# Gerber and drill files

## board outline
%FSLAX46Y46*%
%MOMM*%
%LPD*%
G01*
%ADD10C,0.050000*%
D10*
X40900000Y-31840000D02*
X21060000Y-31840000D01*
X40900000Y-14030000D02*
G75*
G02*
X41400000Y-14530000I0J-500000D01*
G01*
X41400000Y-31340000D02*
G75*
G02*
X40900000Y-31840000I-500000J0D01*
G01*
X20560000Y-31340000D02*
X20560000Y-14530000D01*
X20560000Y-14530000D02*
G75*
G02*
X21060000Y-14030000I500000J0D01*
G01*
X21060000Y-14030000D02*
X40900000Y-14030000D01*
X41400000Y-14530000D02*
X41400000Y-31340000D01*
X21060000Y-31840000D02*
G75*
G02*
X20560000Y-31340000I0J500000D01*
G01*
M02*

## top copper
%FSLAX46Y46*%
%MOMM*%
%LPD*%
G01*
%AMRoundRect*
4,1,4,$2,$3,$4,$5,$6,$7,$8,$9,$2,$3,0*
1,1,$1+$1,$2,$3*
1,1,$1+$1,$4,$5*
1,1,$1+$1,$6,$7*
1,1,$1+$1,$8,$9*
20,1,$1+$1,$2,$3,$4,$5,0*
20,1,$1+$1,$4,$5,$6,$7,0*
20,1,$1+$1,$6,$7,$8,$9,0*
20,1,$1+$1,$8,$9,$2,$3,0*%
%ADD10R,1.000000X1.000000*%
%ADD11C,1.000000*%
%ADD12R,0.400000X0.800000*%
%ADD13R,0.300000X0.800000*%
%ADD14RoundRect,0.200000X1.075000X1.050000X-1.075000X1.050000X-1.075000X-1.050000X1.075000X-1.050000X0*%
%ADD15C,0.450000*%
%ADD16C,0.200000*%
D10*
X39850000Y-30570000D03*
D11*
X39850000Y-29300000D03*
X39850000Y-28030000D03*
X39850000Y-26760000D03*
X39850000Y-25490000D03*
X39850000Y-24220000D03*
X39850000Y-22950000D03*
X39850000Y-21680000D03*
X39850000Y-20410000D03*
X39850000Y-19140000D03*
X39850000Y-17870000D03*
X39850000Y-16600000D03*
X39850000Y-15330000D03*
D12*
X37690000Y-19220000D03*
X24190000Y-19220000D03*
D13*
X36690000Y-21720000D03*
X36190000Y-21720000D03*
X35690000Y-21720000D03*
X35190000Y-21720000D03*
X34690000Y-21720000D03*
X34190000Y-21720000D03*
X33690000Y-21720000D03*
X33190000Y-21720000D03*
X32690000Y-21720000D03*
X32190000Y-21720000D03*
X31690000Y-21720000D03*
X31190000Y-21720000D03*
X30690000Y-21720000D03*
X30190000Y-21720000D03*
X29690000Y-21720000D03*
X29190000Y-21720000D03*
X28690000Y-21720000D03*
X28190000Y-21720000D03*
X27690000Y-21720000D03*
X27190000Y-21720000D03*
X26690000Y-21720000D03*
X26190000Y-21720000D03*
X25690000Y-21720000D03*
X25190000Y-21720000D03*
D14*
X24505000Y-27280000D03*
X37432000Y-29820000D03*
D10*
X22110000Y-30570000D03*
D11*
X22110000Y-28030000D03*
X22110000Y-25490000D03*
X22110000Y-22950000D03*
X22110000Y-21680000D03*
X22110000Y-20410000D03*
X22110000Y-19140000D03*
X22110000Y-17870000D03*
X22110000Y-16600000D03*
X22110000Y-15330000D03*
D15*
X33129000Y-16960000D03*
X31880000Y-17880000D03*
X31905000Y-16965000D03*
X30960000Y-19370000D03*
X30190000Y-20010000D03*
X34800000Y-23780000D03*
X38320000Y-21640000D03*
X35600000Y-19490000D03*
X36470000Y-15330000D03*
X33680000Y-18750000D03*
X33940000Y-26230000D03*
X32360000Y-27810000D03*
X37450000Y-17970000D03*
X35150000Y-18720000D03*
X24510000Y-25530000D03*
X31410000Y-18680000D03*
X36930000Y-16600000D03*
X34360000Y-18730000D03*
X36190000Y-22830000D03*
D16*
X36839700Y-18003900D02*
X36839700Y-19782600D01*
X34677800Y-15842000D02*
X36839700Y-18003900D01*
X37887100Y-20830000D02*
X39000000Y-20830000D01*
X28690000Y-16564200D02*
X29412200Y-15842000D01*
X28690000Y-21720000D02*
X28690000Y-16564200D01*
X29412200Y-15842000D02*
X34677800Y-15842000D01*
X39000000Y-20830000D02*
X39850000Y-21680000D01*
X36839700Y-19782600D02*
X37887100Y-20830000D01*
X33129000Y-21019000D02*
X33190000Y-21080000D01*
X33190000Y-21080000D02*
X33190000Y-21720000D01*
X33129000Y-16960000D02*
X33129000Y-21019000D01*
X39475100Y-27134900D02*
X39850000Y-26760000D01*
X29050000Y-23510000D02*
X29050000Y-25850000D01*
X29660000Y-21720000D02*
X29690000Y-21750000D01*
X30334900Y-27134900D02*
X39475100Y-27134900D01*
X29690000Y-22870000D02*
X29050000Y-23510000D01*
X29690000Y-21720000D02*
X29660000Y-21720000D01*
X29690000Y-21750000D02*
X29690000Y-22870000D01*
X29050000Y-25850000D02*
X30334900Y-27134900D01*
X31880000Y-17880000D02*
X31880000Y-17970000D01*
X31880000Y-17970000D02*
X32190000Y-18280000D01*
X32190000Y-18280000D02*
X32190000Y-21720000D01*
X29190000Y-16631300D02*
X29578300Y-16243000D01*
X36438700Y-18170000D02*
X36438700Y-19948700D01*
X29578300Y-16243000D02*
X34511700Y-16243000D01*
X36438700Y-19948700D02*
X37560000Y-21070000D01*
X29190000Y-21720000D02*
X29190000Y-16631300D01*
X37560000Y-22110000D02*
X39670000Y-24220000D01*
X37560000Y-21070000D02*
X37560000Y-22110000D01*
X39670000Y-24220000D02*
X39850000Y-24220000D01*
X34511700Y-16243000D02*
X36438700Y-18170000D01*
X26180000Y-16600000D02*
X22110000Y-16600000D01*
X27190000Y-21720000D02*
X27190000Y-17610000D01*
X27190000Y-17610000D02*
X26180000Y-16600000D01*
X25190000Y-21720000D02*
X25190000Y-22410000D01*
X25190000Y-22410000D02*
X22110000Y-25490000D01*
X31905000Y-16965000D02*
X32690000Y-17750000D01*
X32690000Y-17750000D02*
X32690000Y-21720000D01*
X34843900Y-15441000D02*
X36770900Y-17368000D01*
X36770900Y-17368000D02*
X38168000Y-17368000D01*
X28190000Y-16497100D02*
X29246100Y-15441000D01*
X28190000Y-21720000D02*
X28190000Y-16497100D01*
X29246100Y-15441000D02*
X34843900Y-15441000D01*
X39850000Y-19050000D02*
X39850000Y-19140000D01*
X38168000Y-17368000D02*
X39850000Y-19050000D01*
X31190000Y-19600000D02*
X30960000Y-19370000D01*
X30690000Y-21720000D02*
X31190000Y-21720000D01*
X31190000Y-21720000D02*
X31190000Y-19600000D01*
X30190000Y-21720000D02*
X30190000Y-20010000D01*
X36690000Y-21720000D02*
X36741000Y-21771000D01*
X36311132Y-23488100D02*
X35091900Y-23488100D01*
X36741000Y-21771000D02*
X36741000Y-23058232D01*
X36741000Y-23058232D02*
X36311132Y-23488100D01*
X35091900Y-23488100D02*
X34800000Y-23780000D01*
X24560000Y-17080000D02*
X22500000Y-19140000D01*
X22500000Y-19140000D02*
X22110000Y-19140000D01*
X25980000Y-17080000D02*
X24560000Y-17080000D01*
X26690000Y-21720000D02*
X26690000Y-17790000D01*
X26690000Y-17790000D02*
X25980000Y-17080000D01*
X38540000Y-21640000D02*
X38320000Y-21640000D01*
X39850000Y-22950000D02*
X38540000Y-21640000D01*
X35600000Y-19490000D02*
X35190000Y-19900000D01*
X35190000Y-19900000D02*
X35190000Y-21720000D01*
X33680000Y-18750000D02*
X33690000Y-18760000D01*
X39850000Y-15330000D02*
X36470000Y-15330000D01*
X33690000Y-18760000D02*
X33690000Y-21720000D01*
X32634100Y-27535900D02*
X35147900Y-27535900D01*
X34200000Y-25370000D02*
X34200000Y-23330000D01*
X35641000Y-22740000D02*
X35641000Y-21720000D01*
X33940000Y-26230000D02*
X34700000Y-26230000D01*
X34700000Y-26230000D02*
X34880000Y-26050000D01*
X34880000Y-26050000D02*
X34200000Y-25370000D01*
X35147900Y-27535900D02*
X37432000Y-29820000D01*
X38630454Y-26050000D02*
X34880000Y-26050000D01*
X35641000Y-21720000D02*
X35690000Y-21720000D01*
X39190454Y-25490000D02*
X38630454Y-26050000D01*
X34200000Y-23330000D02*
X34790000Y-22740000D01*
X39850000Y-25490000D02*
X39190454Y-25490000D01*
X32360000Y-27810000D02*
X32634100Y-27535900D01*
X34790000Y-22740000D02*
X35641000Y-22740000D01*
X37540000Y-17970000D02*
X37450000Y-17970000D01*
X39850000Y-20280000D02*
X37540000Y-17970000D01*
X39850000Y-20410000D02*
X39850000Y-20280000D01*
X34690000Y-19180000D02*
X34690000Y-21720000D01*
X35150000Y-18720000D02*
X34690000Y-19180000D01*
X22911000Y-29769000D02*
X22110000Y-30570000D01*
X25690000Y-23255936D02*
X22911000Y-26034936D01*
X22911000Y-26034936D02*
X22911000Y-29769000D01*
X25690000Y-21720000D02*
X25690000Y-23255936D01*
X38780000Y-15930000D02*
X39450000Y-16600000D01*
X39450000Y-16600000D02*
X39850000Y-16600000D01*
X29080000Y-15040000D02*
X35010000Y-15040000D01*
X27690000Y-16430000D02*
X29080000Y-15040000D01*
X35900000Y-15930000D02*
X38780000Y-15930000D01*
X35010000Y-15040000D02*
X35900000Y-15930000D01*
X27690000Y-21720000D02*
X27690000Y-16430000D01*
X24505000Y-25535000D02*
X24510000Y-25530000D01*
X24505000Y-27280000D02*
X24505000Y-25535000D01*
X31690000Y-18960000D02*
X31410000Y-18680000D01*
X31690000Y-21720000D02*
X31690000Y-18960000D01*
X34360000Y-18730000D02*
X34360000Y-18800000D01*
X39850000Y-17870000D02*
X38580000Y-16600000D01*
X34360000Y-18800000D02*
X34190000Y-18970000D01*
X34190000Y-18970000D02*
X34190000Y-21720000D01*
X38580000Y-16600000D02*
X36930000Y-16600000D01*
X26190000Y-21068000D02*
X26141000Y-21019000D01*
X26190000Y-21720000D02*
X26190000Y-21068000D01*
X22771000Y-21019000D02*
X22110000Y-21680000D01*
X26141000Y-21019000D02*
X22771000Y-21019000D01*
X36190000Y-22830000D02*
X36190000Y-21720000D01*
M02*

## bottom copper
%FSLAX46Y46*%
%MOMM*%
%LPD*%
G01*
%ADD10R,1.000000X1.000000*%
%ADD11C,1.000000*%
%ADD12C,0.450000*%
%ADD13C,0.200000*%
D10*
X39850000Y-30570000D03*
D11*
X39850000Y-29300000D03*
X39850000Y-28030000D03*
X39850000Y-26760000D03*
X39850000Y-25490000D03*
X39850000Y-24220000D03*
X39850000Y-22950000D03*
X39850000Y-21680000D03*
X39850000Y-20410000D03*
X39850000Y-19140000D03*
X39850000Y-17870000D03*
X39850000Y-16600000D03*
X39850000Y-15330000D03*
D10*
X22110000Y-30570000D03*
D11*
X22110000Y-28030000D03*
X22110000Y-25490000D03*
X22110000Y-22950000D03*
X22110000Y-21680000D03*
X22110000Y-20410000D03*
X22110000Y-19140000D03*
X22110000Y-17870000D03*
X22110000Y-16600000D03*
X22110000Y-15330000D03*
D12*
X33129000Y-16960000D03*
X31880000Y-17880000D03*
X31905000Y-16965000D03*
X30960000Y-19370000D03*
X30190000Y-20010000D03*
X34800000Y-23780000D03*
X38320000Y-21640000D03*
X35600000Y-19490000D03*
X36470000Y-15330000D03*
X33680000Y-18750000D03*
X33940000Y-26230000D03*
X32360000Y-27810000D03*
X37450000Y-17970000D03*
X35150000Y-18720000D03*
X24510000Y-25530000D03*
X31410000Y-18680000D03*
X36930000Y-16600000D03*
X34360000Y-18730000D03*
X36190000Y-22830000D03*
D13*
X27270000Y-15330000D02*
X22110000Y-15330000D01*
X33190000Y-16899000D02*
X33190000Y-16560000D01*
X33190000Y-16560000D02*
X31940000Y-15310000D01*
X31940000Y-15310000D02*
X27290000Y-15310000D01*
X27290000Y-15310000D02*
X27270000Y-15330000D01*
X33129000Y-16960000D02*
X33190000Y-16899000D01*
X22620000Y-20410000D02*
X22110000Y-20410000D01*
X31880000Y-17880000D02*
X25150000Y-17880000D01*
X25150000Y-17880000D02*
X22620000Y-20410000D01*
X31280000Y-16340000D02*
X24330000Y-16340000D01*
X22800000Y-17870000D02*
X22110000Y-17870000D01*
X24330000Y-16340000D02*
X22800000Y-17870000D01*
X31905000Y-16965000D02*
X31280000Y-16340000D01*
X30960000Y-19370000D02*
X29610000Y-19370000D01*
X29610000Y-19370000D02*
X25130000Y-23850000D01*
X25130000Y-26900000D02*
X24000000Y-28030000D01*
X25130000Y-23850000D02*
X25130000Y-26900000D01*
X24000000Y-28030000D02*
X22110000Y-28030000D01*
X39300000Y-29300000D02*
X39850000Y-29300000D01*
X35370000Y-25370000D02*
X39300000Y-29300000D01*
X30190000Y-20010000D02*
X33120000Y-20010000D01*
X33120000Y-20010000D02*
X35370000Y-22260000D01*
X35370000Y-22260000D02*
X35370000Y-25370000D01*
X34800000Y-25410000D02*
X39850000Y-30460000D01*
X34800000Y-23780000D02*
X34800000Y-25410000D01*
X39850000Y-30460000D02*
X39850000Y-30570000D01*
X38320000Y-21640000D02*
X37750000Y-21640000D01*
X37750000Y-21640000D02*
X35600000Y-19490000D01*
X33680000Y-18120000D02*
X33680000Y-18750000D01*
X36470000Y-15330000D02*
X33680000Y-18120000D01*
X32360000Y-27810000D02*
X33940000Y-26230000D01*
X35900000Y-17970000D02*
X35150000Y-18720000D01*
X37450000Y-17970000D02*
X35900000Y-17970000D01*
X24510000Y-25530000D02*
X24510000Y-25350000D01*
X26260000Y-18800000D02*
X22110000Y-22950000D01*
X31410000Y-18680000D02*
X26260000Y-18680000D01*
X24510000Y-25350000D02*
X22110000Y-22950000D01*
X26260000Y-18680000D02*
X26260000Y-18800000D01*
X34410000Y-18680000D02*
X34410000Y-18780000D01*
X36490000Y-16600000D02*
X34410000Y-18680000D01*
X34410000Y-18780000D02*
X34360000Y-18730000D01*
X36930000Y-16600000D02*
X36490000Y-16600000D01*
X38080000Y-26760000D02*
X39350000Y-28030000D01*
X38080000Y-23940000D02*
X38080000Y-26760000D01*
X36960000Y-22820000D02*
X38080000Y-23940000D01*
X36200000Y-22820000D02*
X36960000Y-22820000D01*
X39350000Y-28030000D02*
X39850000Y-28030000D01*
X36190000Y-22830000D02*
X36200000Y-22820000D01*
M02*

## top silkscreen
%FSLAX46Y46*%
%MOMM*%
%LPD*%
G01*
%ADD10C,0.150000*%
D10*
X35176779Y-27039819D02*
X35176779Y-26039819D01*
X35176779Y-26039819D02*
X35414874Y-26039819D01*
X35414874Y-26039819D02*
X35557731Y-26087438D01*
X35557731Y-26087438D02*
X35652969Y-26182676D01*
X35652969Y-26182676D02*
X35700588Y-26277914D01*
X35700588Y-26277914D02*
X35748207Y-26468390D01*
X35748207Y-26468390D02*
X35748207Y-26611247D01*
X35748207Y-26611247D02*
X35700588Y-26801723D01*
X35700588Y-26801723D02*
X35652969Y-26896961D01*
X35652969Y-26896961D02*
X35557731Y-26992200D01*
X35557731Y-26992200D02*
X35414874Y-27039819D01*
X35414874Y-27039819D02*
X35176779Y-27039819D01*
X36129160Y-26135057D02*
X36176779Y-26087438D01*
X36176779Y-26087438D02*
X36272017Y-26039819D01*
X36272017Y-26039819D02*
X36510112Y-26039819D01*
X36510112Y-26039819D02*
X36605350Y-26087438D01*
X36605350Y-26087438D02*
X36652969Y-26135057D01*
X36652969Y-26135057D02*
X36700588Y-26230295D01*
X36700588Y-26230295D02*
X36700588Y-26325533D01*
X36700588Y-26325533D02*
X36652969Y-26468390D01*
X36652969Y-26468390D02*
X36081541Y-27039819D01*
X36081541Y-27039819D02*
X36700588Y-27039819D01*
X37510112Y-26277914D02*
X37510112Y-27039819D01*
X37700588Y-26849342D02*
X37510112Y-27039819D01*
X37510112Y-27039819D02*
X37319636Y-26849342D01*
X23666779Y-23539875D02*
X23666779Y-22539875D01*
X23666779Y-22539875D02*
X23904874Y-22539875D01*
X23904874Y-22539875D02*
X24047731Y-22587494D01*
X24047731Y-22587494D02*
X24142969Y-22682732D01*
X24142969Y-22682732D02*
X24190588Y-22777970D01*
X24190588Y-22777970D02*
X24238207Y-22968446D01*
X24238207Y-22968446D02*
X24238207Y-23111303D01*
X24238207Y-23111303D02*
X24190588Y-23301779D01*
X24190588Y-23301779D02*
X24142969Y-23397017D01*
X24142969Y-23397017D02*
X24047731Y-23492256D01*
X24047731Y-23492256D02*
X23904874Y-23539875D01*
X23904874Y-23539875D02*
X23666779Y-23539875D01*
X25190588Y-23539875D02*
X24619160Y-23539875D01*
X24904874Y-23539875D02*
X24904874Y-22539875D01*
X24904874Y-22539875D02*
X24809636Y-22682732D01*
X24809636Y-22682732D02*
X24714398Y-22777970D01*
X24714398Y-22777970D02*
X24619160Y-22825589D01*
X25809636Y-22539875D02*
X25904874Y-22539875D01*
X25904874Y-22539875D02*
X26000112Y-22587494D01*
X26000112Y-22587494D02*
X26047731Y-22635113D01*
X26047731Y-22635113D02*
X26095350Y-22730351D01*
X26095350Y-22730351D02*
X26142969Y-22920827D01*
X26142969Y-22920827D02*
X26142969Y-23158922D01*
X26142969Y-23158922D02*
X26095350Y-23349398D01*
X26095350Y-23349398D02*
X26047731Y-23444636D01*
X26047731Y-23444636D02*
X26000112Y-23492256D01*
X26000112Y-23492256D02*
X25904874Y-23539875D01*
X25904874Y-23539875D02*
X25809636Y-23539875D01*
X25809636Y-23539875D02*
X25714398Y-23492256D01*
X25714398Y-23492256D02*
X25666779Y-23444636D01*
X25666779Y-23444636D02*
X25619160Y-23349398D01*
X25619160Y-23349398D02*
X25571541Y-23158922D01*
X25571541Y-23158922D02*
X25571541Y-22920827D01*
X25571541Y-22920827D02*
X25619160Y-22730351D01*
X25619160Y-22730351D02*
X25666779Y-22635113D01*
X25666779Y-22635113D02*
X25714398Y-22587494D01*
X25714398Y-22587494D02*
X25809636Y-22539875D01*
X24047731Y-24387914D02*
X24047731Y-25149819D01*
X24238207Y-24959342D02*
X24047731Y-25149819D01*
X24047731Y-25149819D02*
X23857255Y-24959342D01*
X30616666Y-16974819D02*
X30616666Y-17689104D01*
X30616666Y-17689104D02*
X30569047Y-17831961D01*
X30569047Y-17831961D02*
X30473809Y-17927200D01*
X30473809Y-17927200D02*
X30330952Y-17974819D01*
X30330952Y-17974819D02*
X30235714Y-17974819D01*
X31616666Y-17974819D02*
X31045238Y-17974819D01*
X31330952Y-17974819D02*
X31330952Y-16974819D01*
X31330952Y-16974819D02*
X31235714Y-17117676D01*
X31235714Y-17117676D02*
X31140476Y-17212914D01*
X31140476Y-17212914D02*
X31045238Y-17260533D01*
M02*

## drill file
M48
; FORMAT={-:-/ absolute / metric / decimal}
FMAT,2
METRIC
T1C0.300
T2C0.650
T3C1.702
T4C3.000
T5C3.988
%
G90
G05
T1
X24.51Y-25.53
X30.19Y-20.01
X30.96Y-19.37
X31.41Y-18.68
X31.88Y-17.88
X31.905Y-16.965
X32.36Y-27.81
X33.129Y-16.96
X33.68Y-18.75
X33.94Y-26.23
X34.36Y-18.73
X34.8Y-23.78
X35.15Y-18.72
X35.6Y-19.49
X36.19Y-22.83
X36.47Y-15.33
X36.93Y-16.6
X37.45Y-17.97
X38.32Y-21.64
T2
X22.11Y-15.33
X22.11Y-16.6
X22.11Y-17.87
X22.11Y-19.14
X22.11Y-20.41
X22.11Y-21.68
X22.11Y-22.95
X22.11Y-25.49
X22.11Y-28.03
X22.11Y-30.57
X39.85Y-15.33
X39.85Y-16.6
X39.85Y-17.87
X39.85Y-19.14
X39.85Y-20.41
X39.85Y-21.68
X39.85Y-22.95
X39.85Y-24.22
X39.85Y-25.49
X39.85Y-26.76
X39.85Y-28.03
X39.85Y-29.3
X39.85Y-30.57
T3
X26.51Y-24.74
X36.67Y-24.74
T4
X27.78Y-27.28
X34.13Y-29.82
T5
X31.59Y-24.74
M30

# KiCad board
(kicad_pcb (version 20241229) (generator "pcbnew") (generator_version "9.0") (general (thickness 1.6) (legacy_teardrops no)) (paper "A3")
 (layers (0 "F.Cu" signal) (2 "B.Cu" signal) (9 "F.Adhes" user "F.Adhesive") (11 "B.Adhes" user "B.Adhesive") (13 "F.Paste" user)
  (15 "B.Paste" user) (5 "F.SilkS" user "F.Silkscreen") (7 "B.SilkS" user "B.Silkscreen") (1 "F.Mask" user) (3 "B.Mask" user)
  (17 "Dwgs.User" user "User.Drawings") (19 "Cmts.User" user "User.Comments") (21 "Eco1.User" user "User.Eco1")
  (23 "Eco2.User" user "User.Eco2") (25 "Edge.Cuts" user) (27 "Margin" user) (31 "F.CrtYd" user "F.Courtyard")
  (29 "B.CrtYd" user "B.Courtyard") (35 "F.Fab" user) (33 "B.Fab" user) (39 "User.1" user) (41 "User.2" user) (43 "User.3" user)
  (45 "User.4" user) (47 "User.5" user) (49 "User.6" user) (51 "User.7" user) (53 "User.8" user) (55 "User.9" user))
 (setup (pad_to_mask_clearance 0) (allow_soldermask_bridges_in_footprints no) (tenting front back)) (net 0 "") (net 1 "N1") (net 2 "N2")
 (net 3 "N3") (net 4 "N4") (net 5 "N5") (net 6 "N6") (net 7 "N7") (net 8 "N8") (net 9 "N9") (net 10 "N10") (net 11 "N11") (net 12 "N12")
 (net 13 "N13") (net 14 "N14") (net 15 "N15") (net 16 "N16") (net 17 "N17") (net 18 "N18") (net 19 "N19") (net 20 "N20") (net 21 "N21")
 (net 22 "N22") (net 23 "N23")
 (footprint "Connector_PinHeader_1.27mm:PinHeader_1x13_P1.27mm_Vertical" (layer "F.Cu") (at 39.85 30.57 180)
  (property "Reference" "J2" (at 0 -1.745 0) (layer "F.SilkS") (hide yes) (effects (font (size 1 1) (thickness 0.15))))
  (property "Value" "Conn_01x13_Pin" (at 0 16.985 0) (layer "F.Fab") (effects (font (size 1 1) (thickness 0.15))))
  (pad "1" thru_hole rect (at 0 0 180) (size 1 1) (drill 0.65) (layers "*.Cu" "*.Mask") (remove_unused_layers no) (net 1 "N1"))
  (pad "2" thru_hole circle (at 0 1.27 180) (size 1 1) (drill 0.65) (layers "*.Cu" "*.Mask") (remove_unused_layers no) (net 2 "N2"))
  (pad "3" thru_hole circle (at 0 2.54 180) (size 1 1) (drill 0.65) (layers "*.Cu" "*.Mask") (remove_unused_layers no) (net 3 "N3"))
  (pad "4" thru_hole circle (at 0 3.81 180) (size 1 1) (drill 0.65) (layers "*.Cu" "*.Mask") (remove_unused_layers no) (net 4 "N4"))
  (pad "5" thru_hole circle (at 0 5.08 180) (size 1 1) (drill 0.65) (layers "*.Cu" "*.Mask") (remove_unused_layers no) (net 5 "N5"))
  (pad "6" thru_hole circle (at 0 6.35 180) (size 1 1) (drill 0.65) (layers "*.Cu" "*.Mask") (remove_unused_layers no) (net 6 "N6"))
  (pad "7" thru_hole circle (at 0 7.62 180) (size 1 1) (drill 0.65) (layers "*.Cu" "*.Mask") (remove_unused_layers no) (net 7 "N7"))
  (pad "8" thru_hole circle (at 0 8.89 180) (size 1 1) (drill 0.65) (layers "*.Cu" "*.Mask") (remove_unused_layers no) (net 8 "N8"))
  (pad "9" thru_hole circle (at 0 10.16 180) (size 1 1) (drill 0.65) (layers "*.Cu" "*.Mask") (remove_unused_layers no) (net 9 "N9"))
  (pad "10" thru_hole circle (at 0 11.43 180) (size 1 1) (drill 0.65) (layers "*.Cu" "*.Mask") (remove_unused_layers no) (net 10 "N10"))
  (pad "11" thru_hole circle (at 0 12.7 180) (size 1 1) (drill 0.65) (layers "*.Cu" "*.Mask") (remove_unused_layers no) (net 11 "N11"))
  (pad "12" thru_hole circle (at 0 13.97 180) (size 1 1) (drill 0.65) (layers "*.Cu" "*.Mask") (remove_unused_layers no) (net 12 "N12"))
  (pad "13" thru_hole circle (at 0 15.24 180) (size 1 1) (drill 0.65) (layers "*.Cu" "*.Mask") (remove_unused_layers no) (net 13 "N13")))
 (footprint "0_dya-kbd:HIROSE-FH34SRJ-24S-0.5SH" (layer "F.Cu") (at 30.94 21.72 180)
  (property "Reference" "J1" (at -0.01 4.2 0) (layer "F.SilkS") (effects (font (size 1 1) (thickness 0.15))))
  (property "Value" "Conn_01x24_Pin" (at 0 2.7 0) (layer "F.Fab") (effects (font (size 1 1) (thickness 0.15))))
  (pad "0" smd rect (at -6.75 2.5 180) (size 0.4 0.8) (layers "F.Cu" "F.Mask" "F.Paste") (thermal_bridge_angle 45))
  (pad "0" smd rect (at 6.75 2.5 180) (size 0.4 0.8) (layers "F.Cu" "F.Mask" "F.Paste") (thermal_bridge_angle 45))
  (pad "1" smd rect (at -5.75 0 180) (size 0.3 0.8) (layers "F.Cu" "F.Mask" "F.Paste") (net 1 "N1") (thermal_bridge_angle 45))
  (pad "2" smd rect (at -5.25 0 180) (size 0.3 0.8) (layers "F.Cu" "F.Mask" "F.Paste") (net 3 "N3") (thermal_bridge_angle 45))
  (pad "3" smd rect (at -4.75 0 180) (size 0.3 0.8) (layers "F.Cu" "F.Mask" "F.Paste") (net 5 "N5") (thermal_bridge_angle 45))
  (pad "4" smd rect (at -4.25 0 180) (size 0.3 0.8) (layers "F.Cu" "F.Mask" "F.Paste") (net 7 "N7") (thermal_bridge_angle 45))
  (pad "5" smd rect (at -3.75 0 180) (size 0.3 0.8) (layers "F.Cu" "F.Mask" "F.Paste") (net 9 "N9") (thermal_bridge_angle 45))
  (pad "6" smd rect (at -3.25 0 180) (size 0.3 0.8) (layers "F.Cu" "F.Mask" "F.Paste") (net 11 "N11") (thermal_bridge_angle 45))
  (pad "7" smd rect (at -2.75 0 180) (size 0.3 0.8) (layers "F.Cu" "F.Mask" "F.Paste") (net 13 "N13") (thermal_bridge_angle 45))
  (pad "8" smd rect (at -2.25 0 180) (size 0.3 0.8) (layers "F.Cu" "F.Mask" "F.Paste") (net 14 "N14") (thermal_bridge_angle 45))
  (pad "9" smd rect (at -1.75 0 180) (size 0.3 0.8) (layers "F.Cu" "F.Mask" "F.Paste") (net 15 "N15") (thermal_bridge_angle 45))
  (pad "10" smd rect (at -1.25 0 180) (size 0.3 0.8) (layers "F.Cu" "F.Mask" "F.Paste") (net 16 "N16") (thermal_bridge_angle 45))
  (pad "11" smd rect (at -0.75 0 180) (size 0.3 0.8) (layers "F.Cu" "F.Mask" "F.Paste") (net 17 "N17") (thermal_bridge_angle 45))
  (pad "12" smd rect (at -0.25 0 180) (size 0.3 0.8) (layers "F.Cu" "F.Mask" "F.Paste") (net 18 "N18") (thermal_bridge_angle 45))
  (pad "13" smd rect (at 0.25 0 180) (size 0.3 0.8) (layers "F.Cu" "F.Mask" "F.Paste") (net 18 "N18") (thermal_bridge_angle 45))
  (pad "14" smd rect (at 0.75 0 180) (size 0.3 0.8) (layers "F.Cu" "F.Mask" "F.Paste") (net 2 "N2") (thermal_bridge_angle 45))
  (pad "15" smd rect (at 1.25 0 180) (size 0.3 0.8) (layers "F.Cu" "F.Mask" "F.Paste") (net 4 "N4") (thermal_bridge_angle 45))
  (pad "16" smd rect (at 1.75 0 180) (size 0.3 0.8) (layers "F.Cu" "F.Mask" "F.Paste") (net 6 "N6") (thermal_bridge_angle 45))
  (pad "17" smd rect (at 2.25 0 180) (size 0.3 0.8) (layers "F.Cu" "F.Mask" "F.Paste") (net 8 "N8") (thermal_bridge_angle 45))
  (pad "18" smd rect (at 2.75 0 180) (size 0.3 0.8) (layers "F.Cu" "F.Mask" "F.Paste") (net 10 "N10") (thermal_bridge_angle 45))
  (pad "19" smd rect (at 3.25 0 180) (size 0.3 0.8) (layers "F.Cu" "F.Mask" "F.Paste") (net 12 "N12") (thermal_bridge_angle 45))
  (pad "20" smd rect (at 3.75 0 180) (size 0.3 0.8) (layers "F.Cu" "F.Mask" "F.Paste") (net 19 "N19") (thermal_bridge_angle 45))
  (pad "21" smd rect (at 4.25 0 180) (size 0.3 0.8) (layers "F.Cu" "F.Mask" "F.Paste") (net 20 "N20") (thermal_bridge_angle 45))
  (pad "22" smd rect (at 4.75 0 180) (size 0.3 0.8) (layers "F.Cu" "F.Mask" "F.Paste") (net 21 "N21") (thermal_bridge_angle 45))
  (pad "23" smd rect (at 5.25 0 180) (size 0.3 0.8) (layers "F.Cu" "F.Mask" "F.Paste") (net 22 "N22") (thermal_bridge_angle 45))
  (pad "24" smd rect (at 5.75 0 180) (size 0.3 0.8) (layers "F.Cu" "F.Mask" "F.Paste") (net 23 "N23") (thermal_bridge_angle 45)))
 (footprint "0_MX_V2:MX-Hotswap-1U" (layer "F.Cu") (at 31.59 24.74 180)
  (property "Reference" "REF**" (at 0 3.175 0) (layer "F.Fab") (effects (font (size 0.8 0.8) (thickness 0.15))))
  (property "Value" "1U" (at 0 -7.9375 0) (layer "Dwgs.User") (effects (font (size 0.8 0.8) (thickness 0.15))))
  (pad "" np_thru_hole circle (at -5.08 0 131.901) (size 1.7018 1.7018) (drill 1.7018) (layers "*.Cu" "*.Mask"))
  (pad "" np_thru_hole circle (at -2.54 -5.08 180) (size 3 3) (drill 3) (layers "*.Cu" "*.Mask"))
  (pad "" np_thru_hole circle (at 0 0 180) (size 3.9878 3.9878) (drill 3.9878) (layers "*.Cu" "*.Mask"))
  (pad "" np_thru_hole circle (at 3.81 -2.54 180) (size 3 3) (drill 3) (layers "*.Cu" "*.Mask"))
  (pad "" np_thru_hole circle (at 5.08 0 131.901) (size 1.7018 1.7018) (drill 1.7018) (layers "*.Cu" "*.Mask"))
  (pad "1" smd roundrect (at 7.085 -2.54 180) (size 2.55 2.5) (layers "F.Cu" "F.Mask" "F.Paste") (roundrect_rratio 0.08) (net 17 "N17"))
  (pad "2" smd roundrect (at -5.842 -5.08 180) (size 2.55 2.5) (layers "F.Cu" "F.Mask" "F.Paste") (roundrect_rratio 0.08) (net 5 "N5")))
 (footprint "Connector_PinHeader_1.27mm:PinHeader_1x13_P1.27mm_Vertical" (layer "F.Cu") (at 22.11 30.57 180)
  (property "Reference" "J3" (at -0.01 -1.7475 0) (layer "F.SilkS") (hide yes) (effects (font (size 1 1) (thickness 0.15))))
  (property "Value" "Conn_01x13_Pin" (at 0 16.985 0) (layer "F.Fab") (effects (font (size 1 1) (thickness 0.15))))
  (pad "1" thru_hole rect (at 0 0 180) (size 1 1) (drill 0.65) (layers "*.Cu" "*.Mask") (remove_unused_layers no) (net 22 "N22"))
  (pad "3" thru_hole circle (at 0 2.54 180) (size 1 1) (drill 0.65) (layers "*.Cu" "*.Mask") (remove_unused_layers no) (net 18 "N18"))
  (pad "5" thru_hole circle (at 0 5.08 180) (size 1 1) (drill 0.65) (layers "*.Cu" "*.Mask") (remove_unused_layers no) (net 23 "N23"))
  (pad "7" thru_hole circle (at 0 7.62 180) (size 1 1) (drill 0.65) (layers "*.Cu" "*.Mask") (remove_unused_layers no) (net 17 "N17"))
  (pad "8" thru_hole circle (at 0 8.89 180) (size 1 1) (drill 0.65) (layers "*.Cu" "*.Mask") (remove_unused_layers no) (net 21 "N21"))
  (pad "9" thru_hole circle (at 0 10.16 180) (size 1 1) (drill 0.65) (layers "*.Cu" "*.Mask") (remove_unused_layers no) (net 16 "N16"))
  (pad "10" thru_hole circle (at 0 11.43 180) (size 1 1) (drill 0.65) (layers "*.Cu" "*.Mask") (remove_unused_layers no) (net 20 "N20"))
  (pad "11" thru_hole circle (at 0 12.7 180) (size 1 1) (drill 0.65) (layers "*.Cu" "*.Mask") (remove_unused_layers no) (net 15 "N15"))
  (pad "12" thru_hole circle (at 0 13.97 180) (size 1 1) (drill 0.65) (layers "*.Cu" "*.Mask") (remove_unused_layers no) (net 19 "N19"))
  (pad "13" thru_hole circle (at 0 15.24 180) (size 1 1) (drill 0.65) (layers "*.Cu" "*.Mask") (remove_unused_layers no) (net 14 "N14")))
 (gr_line (start 40.9 31.84) (end 21.06 31.84) (stroke (width 0.05) (type default)) (layer "Edge.Cuts"))
 (gr_arc (start 40.9 14.03) (mid 41.253553 14.176447) (end 41.4 14.53) (stroke (width 0.05) (type default)) (layer "Edge.Cuts"))
 (gr_arc (start 41.4 31.34) (mid 41.253553 31.693553) (end 40.9 31.84) (stroke (width 0.05) (type default)) (layer "Edge.Cuts"))
 (gr_line (start 20.56 31.34) (end 20.56 14.53) (stroke (width 0.05) (type default)) (layer "Edge.Cuts"))
 (gr_arc (start 20.56 14.53) (mid 20.706447 14.176447) (end 21.06 14.03) (stroke (width 0.05) (type default)) (layer "Edge.Cuts"))
 (gr_line (start 21.06 14.03) (end 40.9 14.03) (stroke (width 0.05) (type default)) (layer "Edge.Cuts"))
 (gr_line (start 41.4 14.53) (end 41.4 31.34) (stroke (width 0.05) (type default)) (layer "Edge.Cuts"))
 (gr_arc (start 21.06 31.84) (mid 20.706447 31.693553) (end 20.56 31.34) (stroke (width 0.05) (type default)) (layer "Edge.Cuts"))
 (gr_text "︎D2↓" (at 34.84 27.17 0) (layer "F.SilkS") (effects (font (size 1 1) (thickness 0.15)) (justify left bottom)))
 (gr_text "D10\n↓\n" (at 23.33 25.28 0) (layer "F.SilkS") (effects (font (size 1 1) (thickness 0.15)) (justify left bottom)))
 (segment (start 36.8397 18.0039) (end 36.8397 19.7826) (width 0.2) (layer "F.Cu") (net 8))
 (segment (start 34.6778 15.842) (end 36.8397 18.0039) (width 0.2) (layer "F.Cu") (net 8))
 (segment (start 37.8871 20.83) (end 39 20.83) (width 0.2) (layer "F.Cu") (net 8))
 (segment (start 28.69 16.5642) (end 29.4122 15.842) (width 0.2) (layer "F.Cu") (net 8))
 (segment (start 28.69 21.72) (end 28.69 16.5642) (width 0.2) (layer "F.Cu") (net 8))
 (segment (start 29.4122 15.842) (end 34.6778 15.842) (width 0.2) (layer "F.Cu") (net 8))
 (segment (start 39 20.83) (end 39.85 21.68) (width 0.2) (layer "F.Cu") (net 8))
 (segment (start 36.8397 19.7826) (end 37.8871 20.83) (width 0.2) (layer "F.Cu") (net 8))
 (segment (start 33.129 21.019) (end 33.19 21.08) (width 0.2) (layer "F.Cu") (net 14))
 (segment (start 33.19 21.08) (end 33.19 21.72) (width 0.2) (layer "F.Cu") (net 14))
 (segment (start 33.129 16.96) (end 33.129 21.019) (width 0.2) (layer "F.Cu") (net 14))
 (via (at 33.129 16.96) (size 0.45) (drill 0.3) (layers "F.Cu" "B.Cu") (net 14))
 (segment (start 27.27 15.33) (end 22.11 15.33) (width 0.2) (layer "B.Cu") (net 14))
 (segment (start 33.19 16.899) (end 33.19 16.56) (width 0.2) (layer "B.Cu") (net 14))
 (segment (start 33.19 16.56) (end 31.94 15.31) (width 0.2) (layer "B.Cu") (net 14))
 (segment (start 31.94 15.31) (end 27.29 15.31) (width 0.2) (layer "B.Cu") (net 14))
 (segment (start 27.29 15.31) (end 27.27 15.33) (width 0.2) (layer "B.Cu") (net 14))
 (segment (start 33.129 16.96) (end 33.19 16.899) (width 0.2) (layer "B.Cu") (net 14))
 (segment (start 39.4751 27.1349) (end 39.85 26.76) (width 0.2) (layer "F.Cu") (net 4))
 (segment (start 29.05 23.51) (end 29.05 25.85) (width 0.2) (layer "F.Cu") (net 4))
 (segment (start 29.66 21.72) (end 29.69 21.75) (width 0.2) (layer "F.Cu") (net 4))
 (segment (start 30.3349 27.1349) (end 39.4751 27.1349) (width 0.2) (layer "F.Cu") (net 4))
 (segment (start 29.69 22.87) (end 29.05 23.51) (width 0.2) (layer "F.Cu") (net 4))
 (segment (start 29.69 21.72) (end 29.66 21.72) (width 0.2) (layer "F.Cu") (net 4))
 (segment (start 29.69 21.75) (end 29.69 22.87) (width 0.2) (layer "F.Cu") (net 4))
 (segment (start 29.05 25.85) (end 30.3349 27.1349) (width 0.2) (layer "F.Cu") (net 4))
 (segment (start 31.88 17.88) (end 31.88 17.97) (width 0.2) (layer "F.Cu") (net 16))
 (segment (start 31.88 17.97) (end 32.19 18.28) (width 0.2) (layer "F.Cu") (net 16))
 (segment (start 32.19 18.28) (end 32.19 21.72) (width 0.2) (layer "F.Cu") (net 16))
 (via (at 31.88 17.88) (size 0.45) (drill 0.3) (layers "F.Cu" "B.Cu") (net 16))
 (segment (start 22.62 20.41) (end 22.11 20.41) (width 0.2) (layer "B.Cu") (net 16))
 (segment (start 31.88 17.88) (end 25.15 17.88) (width 0.2) (layer "B.Cu") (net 16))
 (segment (start 25.15 17.88) (end 22.62 20.41) (width 0.2) (layer "B.Cu") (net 16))
 (segment (start 29.19 16.6313) (end 29.5783 16.243) (width 0.2) (layer "F.Cu") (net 6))
 (segment (start 36.4387 18.17) (end 36.4387 19.9487) (width 0.2) (layer "F.Cu") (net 6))
 (segment (start 29.5783 16.243) (end 34.5117 16.243) (width 0.2) (layer "F.Cu") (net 6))
 (segment (start 36.4387 19.9487) (end 37.56 21.07) (width 0.2) (layer "F.Cu") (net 6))
 (segment (start 29.19 21.72) (end 29.19 16.6313) (width 0.2) (layer "F.Cu") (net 6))
 (segment (start 37.56 22.11) (end 39.67 24.22) (width 0.2) (layer "F.Cu") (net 6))
 (segment (start 37.56 21.07) (end 37.56 22.11) (width 0.2) (layer "F.Cu") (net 6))
 (segment (start 39.67 24.22) (end 39.85 24.22) (width 0.2) (layer "F.Cu") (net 6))
 (segment (start 34.5117 16.243) (end 36.4387 18.17) (width 0.2) (layer "F.Cu") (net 6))
 (segment (start 26.18 16.6) (end 22.11 16.6) (width 0.2) (layer "F.Cu") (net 19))
 (segment (start 27.19 21.72) (end 27.19 17.61) (width 0.2) (layer "F.Cu") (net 19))
 (segment (start 27.19 17.61) (end 26.18 16.6) (width 0.2) (layer "F.Cu") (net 19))
 (segment (start 25.19 21.72) (end 25.19 22.41) (width 0.2) (layer "F.Cu") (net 23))
 (segment (start 25.19 22.41) (end 22.11 25.49) (width 0.2) (layer "F.Cu") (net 23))
 (segment (start 31.905 16.965) (end 32.69 17.75) (width 0.2) (layer "F.Cu") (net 15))
 (segment (start 32.69 17.75) (end 32.69 21.72) (width 0.2) (layer "F.Cu") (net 15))
 (via (at 31.905 16.965) (size 0.45) (drill 0.3) (layers "F.Cu" "B.Cu") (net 15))
 (segment (start 31.28 16.34) (end 24.33 16.34) (width 0.2) (layer "B.Cu") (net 15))
 (segment (start 22.8 17.87) (end 22.11 17.87) (width 0.2) (layer "B.Cu") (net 15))
 (segment (start 24.33 16.34) (end 22.8 17.87) (width 0.2) (layer "B.Cu") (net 15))
 (segment (start 31.905 16.965) (end 31.28 16.34) (width 0.2) (layer "B.Cu") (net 15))
 (segment (start 34.8439 15.441) (end 36.7709 17.368) (width 0.2) (layer "F.Cu") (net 10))
 (segment (start 36.7709 17.368) (end 38.168 17.368) (width 0.2) (layer "F.Cu") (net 10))
 (segment (start 28.19 16.4971) (end 29.2461 15.441) (width 0.2) (layer "F.Cu") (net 10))
 (segment (start 28.19 21.72) (end 28.19 16.4971) (width 0.2) (layer "F.Cu") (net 10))
 (segment (start 29.2461 15.441) (end 34.8439 15.441) (width 0.2) (layer "F.Cu") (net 10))
 (segment (start 39.85 19.05) (end 39.85 19.14) (width 0.2) (layer "F.Cu") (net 10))
 (segment (start 38.168 17.368) (end 39.85 19.05) (width 0.2) (layer "F.Cu") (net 10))
 (segment (start 31.19 19.6) (end 30.96 19.37) (width 0.2) (layer "F.Cu") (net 18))
 (segment (start 30.69 21.72) (end 31.19 21.72) (width 0.2) (layer "F.Cu") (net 18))
 (segment (start 31.19 21.72) (end 31.19 19.6) (width 0.2) (layer "F.Cu") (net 18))
 (via (at 30.96 19.37) (size 0.45) (drill 0.3) (layers "F.Cu" "B.Cu") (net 18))
 (segment (start 30.96 19.37) (end 29.61 19.37) (width 0.2) (layer "B.Cu") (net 18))
 (segment (start 29.61 19.37) (end 25.13 23.85) (width 0.2) (layer "B.Cu") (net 18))
 (segment (start 25.13 26.9) (end 24 28.03) (width 0.2) (layer "B.Cu") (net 18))
 (segment (start 25.13 23.85) (end 25.13 26.9) (width 0.2) (layer "B.Cu") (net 18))
 (segment (start 24 28.03) (end 22.11 28.03) (width 0.2) (layer "B.Cu") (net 18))
 (segment (start 30.19 21.72) (end 30.19 20.01) (width 0.2) (layer "F.Cu") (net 2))
 (via (at 30.19 20.01) (size 0.45) (drill 0.3) (layers "F.Cu" "B.Cu") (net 2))
 (segment (start 39.3 29.3) (end 39.85 29.3) (width 0.2) (layer "B.Cu") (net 2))
 (segment (start 35.37 25.37) (end 39.3 29.3) (width 0.2) (layer "B.Cu") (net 2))
 (segment (start 30.19 20.01) (end 33.12 20.01) (width 0.2) (layer "B.Cu") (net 2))
 (segment (start 33.12 20.01) (end 35.37 22.26) (width 0.2) (layer "B.Cu") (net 2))
 (segment (start 35.37 22.26) (end 35.37 25.37) (width 0.2) (layer "B.Cu") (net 2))
 (segment (start 36.69 21.72) (end 36.741 21.771) (width 0.2) (layer "F.Cu") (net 1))
 (segment (start 36.311132 23.4881) (end 35.0919 23.4881) (width 0.2) (layer "F.Cu") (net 1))
 (segment (start 36.741 21.771) (end 36.741 23.058232) (width 0.2) (layer "F.Cu") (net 1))
 (segment (start 36.741 23.058232) (end 36.311132 23.4881) (width 0.2) (layer "F.Cu") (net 1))
 (segment (start 35.0919 23.4881) (end 34.8 23.78) (width 0.2) (layer "F.Cu") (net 1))
 (via (at 34.8 23.78) (size 0.45) (drill 0.3) (layers "F.Cu" "B.Cu") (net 1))
 (segment (start 34.8 25.41) (end 39.85 30.46) (width 0.2) (layer "B.Cu") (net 1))
 (segment (start 34.8 23.78) (end 34.8 25.41) (width 0.2) (layer "B.Cu") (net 1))
 (segment (start 39.85 30.46) (end 39.85 30.57) (width 0.2) (layer "B.Cu") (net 1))
 (segment (start 24.56 17.08) (end 22.5 19.14) (width 0.2) (layer "F.Cu") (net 20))
 (segment (start 22.5 19.14) (end 22.11 19.14) (width 0.2) (layer "F.Cu") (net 20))
 (segment (start 25.98 17.08) (end 24.56 17.08) (width 0.2) (layer "F.Cu") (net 20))
 (segment (start 26.69 21.72) (end 26.69 17.79) (width 0.2) (layer "F.Cu") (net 20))
 (segment (start 26.69 17.79) (end 25.98 17.08) (width 0.2) (layer "F.Cu") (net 20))
 (segment (start 38.54 21.64) (end 38.32 21.64) (width 0.2) (layer "F.Cu") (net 7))
 (segment (start 39.85 22.95) (end 38.54 21.64) (width 0.2) (layer "F.Cu") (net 7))
 (segment (start 35.6 19.49) (end 35.19 19.9) (width 0.2) (layer "F.Cu") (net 7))
 (segment (start 35.19 19.9) (end 35.19 21.72) (width 0.2) (layer "F.Cu") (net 7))
 (via (at 38.32 21.64) (size 0.45) (drill 0.3) (layers "F.Cu" "B.Cu") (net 7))
 (via (at 35.6 19.49) (size 0.45) (drill 0.3) (layers "F.Cu" "B.Cu") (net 7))
 (segment (start 38.32 21.64) (end 37.75 21.64) (width 0.2) (layer "B.Cu") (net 7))
 (segment (start 37.75 21.64) (end 35.6 19.49) (width 0.2) (layer "B.Cu") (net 7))
 (segment (start 33.68 18.75) (end 33.69 18.76) (width 0.2) (layer "F.Cu") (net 13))
 (segment (start 39.85 15.33) (end 36.47 15.33) (width 0.2) (layer "F.Cu") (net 13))
 (segment (start 33.69 18.76) (end 33.69 21.72) (width 0.2) (layer "F.Cu") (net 13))
 (via (at 36.47 15.33) (size 0.45) (drill 0.3) (layers "F.Cu" "B.Cu") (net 13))
 (via (at 33.68 18.75) (size 0.45) (drill 0.3) (layers "F.Cu" "B.Cu") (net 13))
 (segment (start 33.68 18.12) (end 33.68 18.75) (width 0.2) (layer "B.Cu") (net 13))
 (segment (start 36.47 15.33) (end 33.68 18.12) (width 0.2) (layer "B.Cu") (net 13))
 (segment (start 32.6341 27.5359) (end 35.1479 27.5359) (width 0.2) (layer "F.Cu") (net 5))
 (segment (start 34.2 25.37) (end 34.2 23.33) (width 0.2) (layer "F.Cu") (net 5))
 (segment (start 35.641 22.74) (end 35.641 21.72) (width 0.2) (layer "F.Cu") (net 5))
 (segment (start 33.94 26.23) (end 34.7 26.23) (width 0.2) (layer "F.Cu") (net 5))
 (segment (start 34.7 26.23) (end 34.88 26.05) (width 0.2) (layer "F.Cu") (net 5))
 (segment (start 34.88 26.05) (end 34.2 25.37) (width 0.2) (layer "F.Cu") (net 5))
 (segment (start 35.1479 27.5359) (end 37.432 29.82) (width 0.2) (layer "F.Cu") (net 5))
 (segment (start 38.630454 26.05) (end 34.88 26.05) (width 0.2) (layer "F.Cu") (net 5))
 (segment (start 35.641 21.72) (end 35.69 21.72) (width 0.2) (layer "F.Cu") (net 5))
 (segment (start 39.190454 25.49) (end 38.630454 26.05) (width 0.2) (layer "F.Cu") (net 5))
 (segment (start 34.2 23.33) (end 34.79 22.74) (width 0.2) (layer "F.Cu") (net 5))
 (segment (start 39.85 25.49) (end 39.190454 25.49) (width 0.2) (layer "F.Cu") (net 5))
 (segment (start 32.36 27.81) (end 32.6341 27.5359) (width 0.2) (layer "F.Cu") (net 5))
 (segment (start 34.79 22.74) (end 35.641 22.74) (width 0.2) (layer "F.Cu") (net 5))
 (via (at 33.94 26.23) (size 0.45) (drill 0.3) (layers "F.Cu" "B.Cu") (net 5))
 (via (at 32.36 27.81) (size 0.45) (drill 0.3) (layers "F.Cu" "B.Cu") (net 5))
 (segment (start 32.36 27.81) (end 33.94 26.23) (width 0.2) (layer "B.Cu") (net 5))
 (segment (start 37.54 17.97) (end 37.45 17.97) (width 0.2) (layer "F.Cu") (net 9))
 (segment (start 39.85 20.28) (end 37.54 17.97) (width 0.2) (layer "F.Cu") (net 9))
 (segment (start 39.85 20.41) (end 39.85 20.28) (width 0.2) (layer "F.Cu") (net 9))
 (segment (start 34.69 19.18) (end 34.69 21.72) (width 0.2) (layer "F.Cu") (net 9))
 (segment (start 35.15 18.72) (end 34.69 19.18) (width 0.2) (layer "F.Cu") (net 9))
 (via (at 37.45 17.97) (size 0.45) (drill 0.3) (layers "F.Cu" "B.Cu") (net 9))
 (via (at 35.15 18.72) (size 0.45) (drill 0.3) (layers "F.Cu" "B.Cu") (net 9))
 (segment (start 35.9 17.97) (end 35.15 18.72) (width 0.2) (layer "B.Cu") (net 9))
 (segment (start 37.45 17.97) (end 35.9 17.97) (width 0.2) (layer "B.Cu") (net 9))
 (segment (start 22.911 29.769) (end 22.11 30.57) (width 0.2) (layer "F.Cu") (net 22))
 (segment (start 25.69 23.255936) (end 22.911 26.034936) (width 0.2) (layer "F.Cu") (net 22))
 (segment (start 22.911 26.034936) (end 22.911 29.769) (width 0.2) (layer "F.Cu") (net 22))
 (segment (start 25.69 21.72) (end 25.69 23.255936) (width 0.2) (layer "F.Cu") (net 22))
 (segment (start 38.78 15.93) (end 39.45 16.6) (width 0.2) (layer "F.Cu") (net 12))
 (segment (start 39.45 16.6) (end 39.85 16.6) (width 0.2) (layer "F.Cu") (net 12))
 (segment (start 29.08 15.04) (end 35.01 15.04) (width 0.2) (layer "F.Cu") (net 12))
 (segment (start 27.69 16.43) (end 29.08 15.04) (width 0.2) (layer "F.Cu") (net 12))
 (segment (start 35.9 15.93) (end 38.78 15.93) (width 0.2) (layer "F.Cu") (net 12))
 (segment (start 35.01 15.04) (end 35.9 15.93) (width 0.2) (layer "F.Cu") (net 12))
 (segment (start 27.69 21.72) (end 27.69 16.43) (width 0.2) (layer "F.Cu") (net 12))
 (segment (start 24.505 25.535) (end 24.51 25.53) (width 0.2) (layer "F.Cu") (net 17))
 (segment (start 24.505 27.28) (end 24.505 25.535) (width 0.2) (layer "F.Cu") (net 17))
 (segment (start 31.69 18.96) (end 31.41 18.68) (width 0.2) (layer "F.Cu") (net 17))
 (segment (start 31.69 21.72) (end 31.69 18.96) (width 0.2) (layer "F.Cu") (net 17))
 (via (at 24.51 25.53) (size 0.45) (drill 0.3) (layers "F.Cu" "B.Cu") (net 17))
 (via (at 31.41 18.68) (size 0.45) (drill 0.3) (layers "F.Cu" "B.Cu") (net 17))
 (segment (start 24.51 25.53) (end 24.51 25.35) (width 0.2) (layer "B.Cu") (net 17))
 (segment (start 26.26 18.8) (end 22.11 22.95) (width 0.2) (layer "B.Cu") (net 17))
 (segment (start 31.41 18.68) (end 26.26 18.68) (width 0.2) (layer "B.Cu") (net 17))
 (segment (start 24.51 25.35) (end 22.11 22.95) (width 0.2) (layer "B.Cu") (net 17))
 (segment (start 26.26 18.68) (end 26.26 18.8) (width 0.2) (layer "B.Cu") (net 17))
 (segment (start 34.36 18.73) (end 34.36 18.8) (width 0.2) (layer "F.Cu") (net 11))
 (segment (start 39.85 17.87) (end 38.58 16.6) (width 0.2) (layer "F.Cu") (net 11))
 (segment (start 34.36 18.8) (end 34.19 18.97) (width 0.2) (layer "F.Cu") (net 11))
 (segment (start 34.19 18.97) (end 34.19 21.72) (width 0.2) (layer "F.Cu") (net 11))
 (segment (start 38.58 16.6) (end 36.93 16.6) (width 0.2) (layer "F.Cu") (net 11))
 (via (at 36.93 16.6) (size 0.45) (drill 0.3) (layers "F.Cu" "B.Cu") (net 11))
 (via (at 34.36 18.73) (size 0.45) (drill 0.3) (layers "F.Cu" "B.Cu") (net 11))
 (segment (start 34.41 18.68) (end 34.41 18.78) (width 0.2) (layer "B.Cu") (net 11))
 (segment (start 36.49 16.6) (end 34.41 18.68) (width 0.2) (layer "B.Cu") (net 11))
 (segment (start 34.41 18.78) (end 34.36 18.73) (width 0.2) (layer "B.Cu") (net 11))
 (segment (start 36.93 16.6) (end 36.49 16.6) (width 0.2) (layer "B.Cu") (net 11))
 (segment (start 26.19 21.068) (end 26.141 21.019) (width 0.2) (layer "F.Cu") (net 21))
 (segment (start 26.19 21.72) (end 26.19 21.068) (width 0.2) (layer "F.Cu") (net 21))
 (segment (start 22.771 21.019) (end 22.11 21.68) (width 0.2) (layer "F.Cu") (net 21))
 (segment (start 26.141 21.019) (end 22.771 21.019) (width 0.2) (layer "F.Cu") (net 21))
 (segment (start 36.19 22.83) (end 36.19 21.72) (width 0.2) (layer "F.Cu") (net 3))
 (via (at 36.19 22.83) (size 0.45) (drill 0.3) (layers "F.Cu" "B.Cu") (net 3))
 (segment (start 38.08 26.76) (end 39.35 28.03) (width 0.2) (layer "B.Cu") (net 3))
 (segment (start 38.08 23.94) (end 38.08 26.76) (width 0.2) (layer "B.Cu") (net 3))
 (segment (start 36.96 22.82) (end 38.08 23.94) (width 0.2) (layer "B.Cu") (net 3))
 (segment (start 36.2 22.82) (end 36.96 22.82) (width 0.2) (layer "B.Cu") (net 3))
 (segment (start 39.35 28.03) (end 39.85 28.03) (width 0.2) (layer "B.Cu") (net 3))
 (segment (start 36.19 22.83) (end 36.2 22.82) (width 0.2) (layer "B.Cu") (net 3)))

